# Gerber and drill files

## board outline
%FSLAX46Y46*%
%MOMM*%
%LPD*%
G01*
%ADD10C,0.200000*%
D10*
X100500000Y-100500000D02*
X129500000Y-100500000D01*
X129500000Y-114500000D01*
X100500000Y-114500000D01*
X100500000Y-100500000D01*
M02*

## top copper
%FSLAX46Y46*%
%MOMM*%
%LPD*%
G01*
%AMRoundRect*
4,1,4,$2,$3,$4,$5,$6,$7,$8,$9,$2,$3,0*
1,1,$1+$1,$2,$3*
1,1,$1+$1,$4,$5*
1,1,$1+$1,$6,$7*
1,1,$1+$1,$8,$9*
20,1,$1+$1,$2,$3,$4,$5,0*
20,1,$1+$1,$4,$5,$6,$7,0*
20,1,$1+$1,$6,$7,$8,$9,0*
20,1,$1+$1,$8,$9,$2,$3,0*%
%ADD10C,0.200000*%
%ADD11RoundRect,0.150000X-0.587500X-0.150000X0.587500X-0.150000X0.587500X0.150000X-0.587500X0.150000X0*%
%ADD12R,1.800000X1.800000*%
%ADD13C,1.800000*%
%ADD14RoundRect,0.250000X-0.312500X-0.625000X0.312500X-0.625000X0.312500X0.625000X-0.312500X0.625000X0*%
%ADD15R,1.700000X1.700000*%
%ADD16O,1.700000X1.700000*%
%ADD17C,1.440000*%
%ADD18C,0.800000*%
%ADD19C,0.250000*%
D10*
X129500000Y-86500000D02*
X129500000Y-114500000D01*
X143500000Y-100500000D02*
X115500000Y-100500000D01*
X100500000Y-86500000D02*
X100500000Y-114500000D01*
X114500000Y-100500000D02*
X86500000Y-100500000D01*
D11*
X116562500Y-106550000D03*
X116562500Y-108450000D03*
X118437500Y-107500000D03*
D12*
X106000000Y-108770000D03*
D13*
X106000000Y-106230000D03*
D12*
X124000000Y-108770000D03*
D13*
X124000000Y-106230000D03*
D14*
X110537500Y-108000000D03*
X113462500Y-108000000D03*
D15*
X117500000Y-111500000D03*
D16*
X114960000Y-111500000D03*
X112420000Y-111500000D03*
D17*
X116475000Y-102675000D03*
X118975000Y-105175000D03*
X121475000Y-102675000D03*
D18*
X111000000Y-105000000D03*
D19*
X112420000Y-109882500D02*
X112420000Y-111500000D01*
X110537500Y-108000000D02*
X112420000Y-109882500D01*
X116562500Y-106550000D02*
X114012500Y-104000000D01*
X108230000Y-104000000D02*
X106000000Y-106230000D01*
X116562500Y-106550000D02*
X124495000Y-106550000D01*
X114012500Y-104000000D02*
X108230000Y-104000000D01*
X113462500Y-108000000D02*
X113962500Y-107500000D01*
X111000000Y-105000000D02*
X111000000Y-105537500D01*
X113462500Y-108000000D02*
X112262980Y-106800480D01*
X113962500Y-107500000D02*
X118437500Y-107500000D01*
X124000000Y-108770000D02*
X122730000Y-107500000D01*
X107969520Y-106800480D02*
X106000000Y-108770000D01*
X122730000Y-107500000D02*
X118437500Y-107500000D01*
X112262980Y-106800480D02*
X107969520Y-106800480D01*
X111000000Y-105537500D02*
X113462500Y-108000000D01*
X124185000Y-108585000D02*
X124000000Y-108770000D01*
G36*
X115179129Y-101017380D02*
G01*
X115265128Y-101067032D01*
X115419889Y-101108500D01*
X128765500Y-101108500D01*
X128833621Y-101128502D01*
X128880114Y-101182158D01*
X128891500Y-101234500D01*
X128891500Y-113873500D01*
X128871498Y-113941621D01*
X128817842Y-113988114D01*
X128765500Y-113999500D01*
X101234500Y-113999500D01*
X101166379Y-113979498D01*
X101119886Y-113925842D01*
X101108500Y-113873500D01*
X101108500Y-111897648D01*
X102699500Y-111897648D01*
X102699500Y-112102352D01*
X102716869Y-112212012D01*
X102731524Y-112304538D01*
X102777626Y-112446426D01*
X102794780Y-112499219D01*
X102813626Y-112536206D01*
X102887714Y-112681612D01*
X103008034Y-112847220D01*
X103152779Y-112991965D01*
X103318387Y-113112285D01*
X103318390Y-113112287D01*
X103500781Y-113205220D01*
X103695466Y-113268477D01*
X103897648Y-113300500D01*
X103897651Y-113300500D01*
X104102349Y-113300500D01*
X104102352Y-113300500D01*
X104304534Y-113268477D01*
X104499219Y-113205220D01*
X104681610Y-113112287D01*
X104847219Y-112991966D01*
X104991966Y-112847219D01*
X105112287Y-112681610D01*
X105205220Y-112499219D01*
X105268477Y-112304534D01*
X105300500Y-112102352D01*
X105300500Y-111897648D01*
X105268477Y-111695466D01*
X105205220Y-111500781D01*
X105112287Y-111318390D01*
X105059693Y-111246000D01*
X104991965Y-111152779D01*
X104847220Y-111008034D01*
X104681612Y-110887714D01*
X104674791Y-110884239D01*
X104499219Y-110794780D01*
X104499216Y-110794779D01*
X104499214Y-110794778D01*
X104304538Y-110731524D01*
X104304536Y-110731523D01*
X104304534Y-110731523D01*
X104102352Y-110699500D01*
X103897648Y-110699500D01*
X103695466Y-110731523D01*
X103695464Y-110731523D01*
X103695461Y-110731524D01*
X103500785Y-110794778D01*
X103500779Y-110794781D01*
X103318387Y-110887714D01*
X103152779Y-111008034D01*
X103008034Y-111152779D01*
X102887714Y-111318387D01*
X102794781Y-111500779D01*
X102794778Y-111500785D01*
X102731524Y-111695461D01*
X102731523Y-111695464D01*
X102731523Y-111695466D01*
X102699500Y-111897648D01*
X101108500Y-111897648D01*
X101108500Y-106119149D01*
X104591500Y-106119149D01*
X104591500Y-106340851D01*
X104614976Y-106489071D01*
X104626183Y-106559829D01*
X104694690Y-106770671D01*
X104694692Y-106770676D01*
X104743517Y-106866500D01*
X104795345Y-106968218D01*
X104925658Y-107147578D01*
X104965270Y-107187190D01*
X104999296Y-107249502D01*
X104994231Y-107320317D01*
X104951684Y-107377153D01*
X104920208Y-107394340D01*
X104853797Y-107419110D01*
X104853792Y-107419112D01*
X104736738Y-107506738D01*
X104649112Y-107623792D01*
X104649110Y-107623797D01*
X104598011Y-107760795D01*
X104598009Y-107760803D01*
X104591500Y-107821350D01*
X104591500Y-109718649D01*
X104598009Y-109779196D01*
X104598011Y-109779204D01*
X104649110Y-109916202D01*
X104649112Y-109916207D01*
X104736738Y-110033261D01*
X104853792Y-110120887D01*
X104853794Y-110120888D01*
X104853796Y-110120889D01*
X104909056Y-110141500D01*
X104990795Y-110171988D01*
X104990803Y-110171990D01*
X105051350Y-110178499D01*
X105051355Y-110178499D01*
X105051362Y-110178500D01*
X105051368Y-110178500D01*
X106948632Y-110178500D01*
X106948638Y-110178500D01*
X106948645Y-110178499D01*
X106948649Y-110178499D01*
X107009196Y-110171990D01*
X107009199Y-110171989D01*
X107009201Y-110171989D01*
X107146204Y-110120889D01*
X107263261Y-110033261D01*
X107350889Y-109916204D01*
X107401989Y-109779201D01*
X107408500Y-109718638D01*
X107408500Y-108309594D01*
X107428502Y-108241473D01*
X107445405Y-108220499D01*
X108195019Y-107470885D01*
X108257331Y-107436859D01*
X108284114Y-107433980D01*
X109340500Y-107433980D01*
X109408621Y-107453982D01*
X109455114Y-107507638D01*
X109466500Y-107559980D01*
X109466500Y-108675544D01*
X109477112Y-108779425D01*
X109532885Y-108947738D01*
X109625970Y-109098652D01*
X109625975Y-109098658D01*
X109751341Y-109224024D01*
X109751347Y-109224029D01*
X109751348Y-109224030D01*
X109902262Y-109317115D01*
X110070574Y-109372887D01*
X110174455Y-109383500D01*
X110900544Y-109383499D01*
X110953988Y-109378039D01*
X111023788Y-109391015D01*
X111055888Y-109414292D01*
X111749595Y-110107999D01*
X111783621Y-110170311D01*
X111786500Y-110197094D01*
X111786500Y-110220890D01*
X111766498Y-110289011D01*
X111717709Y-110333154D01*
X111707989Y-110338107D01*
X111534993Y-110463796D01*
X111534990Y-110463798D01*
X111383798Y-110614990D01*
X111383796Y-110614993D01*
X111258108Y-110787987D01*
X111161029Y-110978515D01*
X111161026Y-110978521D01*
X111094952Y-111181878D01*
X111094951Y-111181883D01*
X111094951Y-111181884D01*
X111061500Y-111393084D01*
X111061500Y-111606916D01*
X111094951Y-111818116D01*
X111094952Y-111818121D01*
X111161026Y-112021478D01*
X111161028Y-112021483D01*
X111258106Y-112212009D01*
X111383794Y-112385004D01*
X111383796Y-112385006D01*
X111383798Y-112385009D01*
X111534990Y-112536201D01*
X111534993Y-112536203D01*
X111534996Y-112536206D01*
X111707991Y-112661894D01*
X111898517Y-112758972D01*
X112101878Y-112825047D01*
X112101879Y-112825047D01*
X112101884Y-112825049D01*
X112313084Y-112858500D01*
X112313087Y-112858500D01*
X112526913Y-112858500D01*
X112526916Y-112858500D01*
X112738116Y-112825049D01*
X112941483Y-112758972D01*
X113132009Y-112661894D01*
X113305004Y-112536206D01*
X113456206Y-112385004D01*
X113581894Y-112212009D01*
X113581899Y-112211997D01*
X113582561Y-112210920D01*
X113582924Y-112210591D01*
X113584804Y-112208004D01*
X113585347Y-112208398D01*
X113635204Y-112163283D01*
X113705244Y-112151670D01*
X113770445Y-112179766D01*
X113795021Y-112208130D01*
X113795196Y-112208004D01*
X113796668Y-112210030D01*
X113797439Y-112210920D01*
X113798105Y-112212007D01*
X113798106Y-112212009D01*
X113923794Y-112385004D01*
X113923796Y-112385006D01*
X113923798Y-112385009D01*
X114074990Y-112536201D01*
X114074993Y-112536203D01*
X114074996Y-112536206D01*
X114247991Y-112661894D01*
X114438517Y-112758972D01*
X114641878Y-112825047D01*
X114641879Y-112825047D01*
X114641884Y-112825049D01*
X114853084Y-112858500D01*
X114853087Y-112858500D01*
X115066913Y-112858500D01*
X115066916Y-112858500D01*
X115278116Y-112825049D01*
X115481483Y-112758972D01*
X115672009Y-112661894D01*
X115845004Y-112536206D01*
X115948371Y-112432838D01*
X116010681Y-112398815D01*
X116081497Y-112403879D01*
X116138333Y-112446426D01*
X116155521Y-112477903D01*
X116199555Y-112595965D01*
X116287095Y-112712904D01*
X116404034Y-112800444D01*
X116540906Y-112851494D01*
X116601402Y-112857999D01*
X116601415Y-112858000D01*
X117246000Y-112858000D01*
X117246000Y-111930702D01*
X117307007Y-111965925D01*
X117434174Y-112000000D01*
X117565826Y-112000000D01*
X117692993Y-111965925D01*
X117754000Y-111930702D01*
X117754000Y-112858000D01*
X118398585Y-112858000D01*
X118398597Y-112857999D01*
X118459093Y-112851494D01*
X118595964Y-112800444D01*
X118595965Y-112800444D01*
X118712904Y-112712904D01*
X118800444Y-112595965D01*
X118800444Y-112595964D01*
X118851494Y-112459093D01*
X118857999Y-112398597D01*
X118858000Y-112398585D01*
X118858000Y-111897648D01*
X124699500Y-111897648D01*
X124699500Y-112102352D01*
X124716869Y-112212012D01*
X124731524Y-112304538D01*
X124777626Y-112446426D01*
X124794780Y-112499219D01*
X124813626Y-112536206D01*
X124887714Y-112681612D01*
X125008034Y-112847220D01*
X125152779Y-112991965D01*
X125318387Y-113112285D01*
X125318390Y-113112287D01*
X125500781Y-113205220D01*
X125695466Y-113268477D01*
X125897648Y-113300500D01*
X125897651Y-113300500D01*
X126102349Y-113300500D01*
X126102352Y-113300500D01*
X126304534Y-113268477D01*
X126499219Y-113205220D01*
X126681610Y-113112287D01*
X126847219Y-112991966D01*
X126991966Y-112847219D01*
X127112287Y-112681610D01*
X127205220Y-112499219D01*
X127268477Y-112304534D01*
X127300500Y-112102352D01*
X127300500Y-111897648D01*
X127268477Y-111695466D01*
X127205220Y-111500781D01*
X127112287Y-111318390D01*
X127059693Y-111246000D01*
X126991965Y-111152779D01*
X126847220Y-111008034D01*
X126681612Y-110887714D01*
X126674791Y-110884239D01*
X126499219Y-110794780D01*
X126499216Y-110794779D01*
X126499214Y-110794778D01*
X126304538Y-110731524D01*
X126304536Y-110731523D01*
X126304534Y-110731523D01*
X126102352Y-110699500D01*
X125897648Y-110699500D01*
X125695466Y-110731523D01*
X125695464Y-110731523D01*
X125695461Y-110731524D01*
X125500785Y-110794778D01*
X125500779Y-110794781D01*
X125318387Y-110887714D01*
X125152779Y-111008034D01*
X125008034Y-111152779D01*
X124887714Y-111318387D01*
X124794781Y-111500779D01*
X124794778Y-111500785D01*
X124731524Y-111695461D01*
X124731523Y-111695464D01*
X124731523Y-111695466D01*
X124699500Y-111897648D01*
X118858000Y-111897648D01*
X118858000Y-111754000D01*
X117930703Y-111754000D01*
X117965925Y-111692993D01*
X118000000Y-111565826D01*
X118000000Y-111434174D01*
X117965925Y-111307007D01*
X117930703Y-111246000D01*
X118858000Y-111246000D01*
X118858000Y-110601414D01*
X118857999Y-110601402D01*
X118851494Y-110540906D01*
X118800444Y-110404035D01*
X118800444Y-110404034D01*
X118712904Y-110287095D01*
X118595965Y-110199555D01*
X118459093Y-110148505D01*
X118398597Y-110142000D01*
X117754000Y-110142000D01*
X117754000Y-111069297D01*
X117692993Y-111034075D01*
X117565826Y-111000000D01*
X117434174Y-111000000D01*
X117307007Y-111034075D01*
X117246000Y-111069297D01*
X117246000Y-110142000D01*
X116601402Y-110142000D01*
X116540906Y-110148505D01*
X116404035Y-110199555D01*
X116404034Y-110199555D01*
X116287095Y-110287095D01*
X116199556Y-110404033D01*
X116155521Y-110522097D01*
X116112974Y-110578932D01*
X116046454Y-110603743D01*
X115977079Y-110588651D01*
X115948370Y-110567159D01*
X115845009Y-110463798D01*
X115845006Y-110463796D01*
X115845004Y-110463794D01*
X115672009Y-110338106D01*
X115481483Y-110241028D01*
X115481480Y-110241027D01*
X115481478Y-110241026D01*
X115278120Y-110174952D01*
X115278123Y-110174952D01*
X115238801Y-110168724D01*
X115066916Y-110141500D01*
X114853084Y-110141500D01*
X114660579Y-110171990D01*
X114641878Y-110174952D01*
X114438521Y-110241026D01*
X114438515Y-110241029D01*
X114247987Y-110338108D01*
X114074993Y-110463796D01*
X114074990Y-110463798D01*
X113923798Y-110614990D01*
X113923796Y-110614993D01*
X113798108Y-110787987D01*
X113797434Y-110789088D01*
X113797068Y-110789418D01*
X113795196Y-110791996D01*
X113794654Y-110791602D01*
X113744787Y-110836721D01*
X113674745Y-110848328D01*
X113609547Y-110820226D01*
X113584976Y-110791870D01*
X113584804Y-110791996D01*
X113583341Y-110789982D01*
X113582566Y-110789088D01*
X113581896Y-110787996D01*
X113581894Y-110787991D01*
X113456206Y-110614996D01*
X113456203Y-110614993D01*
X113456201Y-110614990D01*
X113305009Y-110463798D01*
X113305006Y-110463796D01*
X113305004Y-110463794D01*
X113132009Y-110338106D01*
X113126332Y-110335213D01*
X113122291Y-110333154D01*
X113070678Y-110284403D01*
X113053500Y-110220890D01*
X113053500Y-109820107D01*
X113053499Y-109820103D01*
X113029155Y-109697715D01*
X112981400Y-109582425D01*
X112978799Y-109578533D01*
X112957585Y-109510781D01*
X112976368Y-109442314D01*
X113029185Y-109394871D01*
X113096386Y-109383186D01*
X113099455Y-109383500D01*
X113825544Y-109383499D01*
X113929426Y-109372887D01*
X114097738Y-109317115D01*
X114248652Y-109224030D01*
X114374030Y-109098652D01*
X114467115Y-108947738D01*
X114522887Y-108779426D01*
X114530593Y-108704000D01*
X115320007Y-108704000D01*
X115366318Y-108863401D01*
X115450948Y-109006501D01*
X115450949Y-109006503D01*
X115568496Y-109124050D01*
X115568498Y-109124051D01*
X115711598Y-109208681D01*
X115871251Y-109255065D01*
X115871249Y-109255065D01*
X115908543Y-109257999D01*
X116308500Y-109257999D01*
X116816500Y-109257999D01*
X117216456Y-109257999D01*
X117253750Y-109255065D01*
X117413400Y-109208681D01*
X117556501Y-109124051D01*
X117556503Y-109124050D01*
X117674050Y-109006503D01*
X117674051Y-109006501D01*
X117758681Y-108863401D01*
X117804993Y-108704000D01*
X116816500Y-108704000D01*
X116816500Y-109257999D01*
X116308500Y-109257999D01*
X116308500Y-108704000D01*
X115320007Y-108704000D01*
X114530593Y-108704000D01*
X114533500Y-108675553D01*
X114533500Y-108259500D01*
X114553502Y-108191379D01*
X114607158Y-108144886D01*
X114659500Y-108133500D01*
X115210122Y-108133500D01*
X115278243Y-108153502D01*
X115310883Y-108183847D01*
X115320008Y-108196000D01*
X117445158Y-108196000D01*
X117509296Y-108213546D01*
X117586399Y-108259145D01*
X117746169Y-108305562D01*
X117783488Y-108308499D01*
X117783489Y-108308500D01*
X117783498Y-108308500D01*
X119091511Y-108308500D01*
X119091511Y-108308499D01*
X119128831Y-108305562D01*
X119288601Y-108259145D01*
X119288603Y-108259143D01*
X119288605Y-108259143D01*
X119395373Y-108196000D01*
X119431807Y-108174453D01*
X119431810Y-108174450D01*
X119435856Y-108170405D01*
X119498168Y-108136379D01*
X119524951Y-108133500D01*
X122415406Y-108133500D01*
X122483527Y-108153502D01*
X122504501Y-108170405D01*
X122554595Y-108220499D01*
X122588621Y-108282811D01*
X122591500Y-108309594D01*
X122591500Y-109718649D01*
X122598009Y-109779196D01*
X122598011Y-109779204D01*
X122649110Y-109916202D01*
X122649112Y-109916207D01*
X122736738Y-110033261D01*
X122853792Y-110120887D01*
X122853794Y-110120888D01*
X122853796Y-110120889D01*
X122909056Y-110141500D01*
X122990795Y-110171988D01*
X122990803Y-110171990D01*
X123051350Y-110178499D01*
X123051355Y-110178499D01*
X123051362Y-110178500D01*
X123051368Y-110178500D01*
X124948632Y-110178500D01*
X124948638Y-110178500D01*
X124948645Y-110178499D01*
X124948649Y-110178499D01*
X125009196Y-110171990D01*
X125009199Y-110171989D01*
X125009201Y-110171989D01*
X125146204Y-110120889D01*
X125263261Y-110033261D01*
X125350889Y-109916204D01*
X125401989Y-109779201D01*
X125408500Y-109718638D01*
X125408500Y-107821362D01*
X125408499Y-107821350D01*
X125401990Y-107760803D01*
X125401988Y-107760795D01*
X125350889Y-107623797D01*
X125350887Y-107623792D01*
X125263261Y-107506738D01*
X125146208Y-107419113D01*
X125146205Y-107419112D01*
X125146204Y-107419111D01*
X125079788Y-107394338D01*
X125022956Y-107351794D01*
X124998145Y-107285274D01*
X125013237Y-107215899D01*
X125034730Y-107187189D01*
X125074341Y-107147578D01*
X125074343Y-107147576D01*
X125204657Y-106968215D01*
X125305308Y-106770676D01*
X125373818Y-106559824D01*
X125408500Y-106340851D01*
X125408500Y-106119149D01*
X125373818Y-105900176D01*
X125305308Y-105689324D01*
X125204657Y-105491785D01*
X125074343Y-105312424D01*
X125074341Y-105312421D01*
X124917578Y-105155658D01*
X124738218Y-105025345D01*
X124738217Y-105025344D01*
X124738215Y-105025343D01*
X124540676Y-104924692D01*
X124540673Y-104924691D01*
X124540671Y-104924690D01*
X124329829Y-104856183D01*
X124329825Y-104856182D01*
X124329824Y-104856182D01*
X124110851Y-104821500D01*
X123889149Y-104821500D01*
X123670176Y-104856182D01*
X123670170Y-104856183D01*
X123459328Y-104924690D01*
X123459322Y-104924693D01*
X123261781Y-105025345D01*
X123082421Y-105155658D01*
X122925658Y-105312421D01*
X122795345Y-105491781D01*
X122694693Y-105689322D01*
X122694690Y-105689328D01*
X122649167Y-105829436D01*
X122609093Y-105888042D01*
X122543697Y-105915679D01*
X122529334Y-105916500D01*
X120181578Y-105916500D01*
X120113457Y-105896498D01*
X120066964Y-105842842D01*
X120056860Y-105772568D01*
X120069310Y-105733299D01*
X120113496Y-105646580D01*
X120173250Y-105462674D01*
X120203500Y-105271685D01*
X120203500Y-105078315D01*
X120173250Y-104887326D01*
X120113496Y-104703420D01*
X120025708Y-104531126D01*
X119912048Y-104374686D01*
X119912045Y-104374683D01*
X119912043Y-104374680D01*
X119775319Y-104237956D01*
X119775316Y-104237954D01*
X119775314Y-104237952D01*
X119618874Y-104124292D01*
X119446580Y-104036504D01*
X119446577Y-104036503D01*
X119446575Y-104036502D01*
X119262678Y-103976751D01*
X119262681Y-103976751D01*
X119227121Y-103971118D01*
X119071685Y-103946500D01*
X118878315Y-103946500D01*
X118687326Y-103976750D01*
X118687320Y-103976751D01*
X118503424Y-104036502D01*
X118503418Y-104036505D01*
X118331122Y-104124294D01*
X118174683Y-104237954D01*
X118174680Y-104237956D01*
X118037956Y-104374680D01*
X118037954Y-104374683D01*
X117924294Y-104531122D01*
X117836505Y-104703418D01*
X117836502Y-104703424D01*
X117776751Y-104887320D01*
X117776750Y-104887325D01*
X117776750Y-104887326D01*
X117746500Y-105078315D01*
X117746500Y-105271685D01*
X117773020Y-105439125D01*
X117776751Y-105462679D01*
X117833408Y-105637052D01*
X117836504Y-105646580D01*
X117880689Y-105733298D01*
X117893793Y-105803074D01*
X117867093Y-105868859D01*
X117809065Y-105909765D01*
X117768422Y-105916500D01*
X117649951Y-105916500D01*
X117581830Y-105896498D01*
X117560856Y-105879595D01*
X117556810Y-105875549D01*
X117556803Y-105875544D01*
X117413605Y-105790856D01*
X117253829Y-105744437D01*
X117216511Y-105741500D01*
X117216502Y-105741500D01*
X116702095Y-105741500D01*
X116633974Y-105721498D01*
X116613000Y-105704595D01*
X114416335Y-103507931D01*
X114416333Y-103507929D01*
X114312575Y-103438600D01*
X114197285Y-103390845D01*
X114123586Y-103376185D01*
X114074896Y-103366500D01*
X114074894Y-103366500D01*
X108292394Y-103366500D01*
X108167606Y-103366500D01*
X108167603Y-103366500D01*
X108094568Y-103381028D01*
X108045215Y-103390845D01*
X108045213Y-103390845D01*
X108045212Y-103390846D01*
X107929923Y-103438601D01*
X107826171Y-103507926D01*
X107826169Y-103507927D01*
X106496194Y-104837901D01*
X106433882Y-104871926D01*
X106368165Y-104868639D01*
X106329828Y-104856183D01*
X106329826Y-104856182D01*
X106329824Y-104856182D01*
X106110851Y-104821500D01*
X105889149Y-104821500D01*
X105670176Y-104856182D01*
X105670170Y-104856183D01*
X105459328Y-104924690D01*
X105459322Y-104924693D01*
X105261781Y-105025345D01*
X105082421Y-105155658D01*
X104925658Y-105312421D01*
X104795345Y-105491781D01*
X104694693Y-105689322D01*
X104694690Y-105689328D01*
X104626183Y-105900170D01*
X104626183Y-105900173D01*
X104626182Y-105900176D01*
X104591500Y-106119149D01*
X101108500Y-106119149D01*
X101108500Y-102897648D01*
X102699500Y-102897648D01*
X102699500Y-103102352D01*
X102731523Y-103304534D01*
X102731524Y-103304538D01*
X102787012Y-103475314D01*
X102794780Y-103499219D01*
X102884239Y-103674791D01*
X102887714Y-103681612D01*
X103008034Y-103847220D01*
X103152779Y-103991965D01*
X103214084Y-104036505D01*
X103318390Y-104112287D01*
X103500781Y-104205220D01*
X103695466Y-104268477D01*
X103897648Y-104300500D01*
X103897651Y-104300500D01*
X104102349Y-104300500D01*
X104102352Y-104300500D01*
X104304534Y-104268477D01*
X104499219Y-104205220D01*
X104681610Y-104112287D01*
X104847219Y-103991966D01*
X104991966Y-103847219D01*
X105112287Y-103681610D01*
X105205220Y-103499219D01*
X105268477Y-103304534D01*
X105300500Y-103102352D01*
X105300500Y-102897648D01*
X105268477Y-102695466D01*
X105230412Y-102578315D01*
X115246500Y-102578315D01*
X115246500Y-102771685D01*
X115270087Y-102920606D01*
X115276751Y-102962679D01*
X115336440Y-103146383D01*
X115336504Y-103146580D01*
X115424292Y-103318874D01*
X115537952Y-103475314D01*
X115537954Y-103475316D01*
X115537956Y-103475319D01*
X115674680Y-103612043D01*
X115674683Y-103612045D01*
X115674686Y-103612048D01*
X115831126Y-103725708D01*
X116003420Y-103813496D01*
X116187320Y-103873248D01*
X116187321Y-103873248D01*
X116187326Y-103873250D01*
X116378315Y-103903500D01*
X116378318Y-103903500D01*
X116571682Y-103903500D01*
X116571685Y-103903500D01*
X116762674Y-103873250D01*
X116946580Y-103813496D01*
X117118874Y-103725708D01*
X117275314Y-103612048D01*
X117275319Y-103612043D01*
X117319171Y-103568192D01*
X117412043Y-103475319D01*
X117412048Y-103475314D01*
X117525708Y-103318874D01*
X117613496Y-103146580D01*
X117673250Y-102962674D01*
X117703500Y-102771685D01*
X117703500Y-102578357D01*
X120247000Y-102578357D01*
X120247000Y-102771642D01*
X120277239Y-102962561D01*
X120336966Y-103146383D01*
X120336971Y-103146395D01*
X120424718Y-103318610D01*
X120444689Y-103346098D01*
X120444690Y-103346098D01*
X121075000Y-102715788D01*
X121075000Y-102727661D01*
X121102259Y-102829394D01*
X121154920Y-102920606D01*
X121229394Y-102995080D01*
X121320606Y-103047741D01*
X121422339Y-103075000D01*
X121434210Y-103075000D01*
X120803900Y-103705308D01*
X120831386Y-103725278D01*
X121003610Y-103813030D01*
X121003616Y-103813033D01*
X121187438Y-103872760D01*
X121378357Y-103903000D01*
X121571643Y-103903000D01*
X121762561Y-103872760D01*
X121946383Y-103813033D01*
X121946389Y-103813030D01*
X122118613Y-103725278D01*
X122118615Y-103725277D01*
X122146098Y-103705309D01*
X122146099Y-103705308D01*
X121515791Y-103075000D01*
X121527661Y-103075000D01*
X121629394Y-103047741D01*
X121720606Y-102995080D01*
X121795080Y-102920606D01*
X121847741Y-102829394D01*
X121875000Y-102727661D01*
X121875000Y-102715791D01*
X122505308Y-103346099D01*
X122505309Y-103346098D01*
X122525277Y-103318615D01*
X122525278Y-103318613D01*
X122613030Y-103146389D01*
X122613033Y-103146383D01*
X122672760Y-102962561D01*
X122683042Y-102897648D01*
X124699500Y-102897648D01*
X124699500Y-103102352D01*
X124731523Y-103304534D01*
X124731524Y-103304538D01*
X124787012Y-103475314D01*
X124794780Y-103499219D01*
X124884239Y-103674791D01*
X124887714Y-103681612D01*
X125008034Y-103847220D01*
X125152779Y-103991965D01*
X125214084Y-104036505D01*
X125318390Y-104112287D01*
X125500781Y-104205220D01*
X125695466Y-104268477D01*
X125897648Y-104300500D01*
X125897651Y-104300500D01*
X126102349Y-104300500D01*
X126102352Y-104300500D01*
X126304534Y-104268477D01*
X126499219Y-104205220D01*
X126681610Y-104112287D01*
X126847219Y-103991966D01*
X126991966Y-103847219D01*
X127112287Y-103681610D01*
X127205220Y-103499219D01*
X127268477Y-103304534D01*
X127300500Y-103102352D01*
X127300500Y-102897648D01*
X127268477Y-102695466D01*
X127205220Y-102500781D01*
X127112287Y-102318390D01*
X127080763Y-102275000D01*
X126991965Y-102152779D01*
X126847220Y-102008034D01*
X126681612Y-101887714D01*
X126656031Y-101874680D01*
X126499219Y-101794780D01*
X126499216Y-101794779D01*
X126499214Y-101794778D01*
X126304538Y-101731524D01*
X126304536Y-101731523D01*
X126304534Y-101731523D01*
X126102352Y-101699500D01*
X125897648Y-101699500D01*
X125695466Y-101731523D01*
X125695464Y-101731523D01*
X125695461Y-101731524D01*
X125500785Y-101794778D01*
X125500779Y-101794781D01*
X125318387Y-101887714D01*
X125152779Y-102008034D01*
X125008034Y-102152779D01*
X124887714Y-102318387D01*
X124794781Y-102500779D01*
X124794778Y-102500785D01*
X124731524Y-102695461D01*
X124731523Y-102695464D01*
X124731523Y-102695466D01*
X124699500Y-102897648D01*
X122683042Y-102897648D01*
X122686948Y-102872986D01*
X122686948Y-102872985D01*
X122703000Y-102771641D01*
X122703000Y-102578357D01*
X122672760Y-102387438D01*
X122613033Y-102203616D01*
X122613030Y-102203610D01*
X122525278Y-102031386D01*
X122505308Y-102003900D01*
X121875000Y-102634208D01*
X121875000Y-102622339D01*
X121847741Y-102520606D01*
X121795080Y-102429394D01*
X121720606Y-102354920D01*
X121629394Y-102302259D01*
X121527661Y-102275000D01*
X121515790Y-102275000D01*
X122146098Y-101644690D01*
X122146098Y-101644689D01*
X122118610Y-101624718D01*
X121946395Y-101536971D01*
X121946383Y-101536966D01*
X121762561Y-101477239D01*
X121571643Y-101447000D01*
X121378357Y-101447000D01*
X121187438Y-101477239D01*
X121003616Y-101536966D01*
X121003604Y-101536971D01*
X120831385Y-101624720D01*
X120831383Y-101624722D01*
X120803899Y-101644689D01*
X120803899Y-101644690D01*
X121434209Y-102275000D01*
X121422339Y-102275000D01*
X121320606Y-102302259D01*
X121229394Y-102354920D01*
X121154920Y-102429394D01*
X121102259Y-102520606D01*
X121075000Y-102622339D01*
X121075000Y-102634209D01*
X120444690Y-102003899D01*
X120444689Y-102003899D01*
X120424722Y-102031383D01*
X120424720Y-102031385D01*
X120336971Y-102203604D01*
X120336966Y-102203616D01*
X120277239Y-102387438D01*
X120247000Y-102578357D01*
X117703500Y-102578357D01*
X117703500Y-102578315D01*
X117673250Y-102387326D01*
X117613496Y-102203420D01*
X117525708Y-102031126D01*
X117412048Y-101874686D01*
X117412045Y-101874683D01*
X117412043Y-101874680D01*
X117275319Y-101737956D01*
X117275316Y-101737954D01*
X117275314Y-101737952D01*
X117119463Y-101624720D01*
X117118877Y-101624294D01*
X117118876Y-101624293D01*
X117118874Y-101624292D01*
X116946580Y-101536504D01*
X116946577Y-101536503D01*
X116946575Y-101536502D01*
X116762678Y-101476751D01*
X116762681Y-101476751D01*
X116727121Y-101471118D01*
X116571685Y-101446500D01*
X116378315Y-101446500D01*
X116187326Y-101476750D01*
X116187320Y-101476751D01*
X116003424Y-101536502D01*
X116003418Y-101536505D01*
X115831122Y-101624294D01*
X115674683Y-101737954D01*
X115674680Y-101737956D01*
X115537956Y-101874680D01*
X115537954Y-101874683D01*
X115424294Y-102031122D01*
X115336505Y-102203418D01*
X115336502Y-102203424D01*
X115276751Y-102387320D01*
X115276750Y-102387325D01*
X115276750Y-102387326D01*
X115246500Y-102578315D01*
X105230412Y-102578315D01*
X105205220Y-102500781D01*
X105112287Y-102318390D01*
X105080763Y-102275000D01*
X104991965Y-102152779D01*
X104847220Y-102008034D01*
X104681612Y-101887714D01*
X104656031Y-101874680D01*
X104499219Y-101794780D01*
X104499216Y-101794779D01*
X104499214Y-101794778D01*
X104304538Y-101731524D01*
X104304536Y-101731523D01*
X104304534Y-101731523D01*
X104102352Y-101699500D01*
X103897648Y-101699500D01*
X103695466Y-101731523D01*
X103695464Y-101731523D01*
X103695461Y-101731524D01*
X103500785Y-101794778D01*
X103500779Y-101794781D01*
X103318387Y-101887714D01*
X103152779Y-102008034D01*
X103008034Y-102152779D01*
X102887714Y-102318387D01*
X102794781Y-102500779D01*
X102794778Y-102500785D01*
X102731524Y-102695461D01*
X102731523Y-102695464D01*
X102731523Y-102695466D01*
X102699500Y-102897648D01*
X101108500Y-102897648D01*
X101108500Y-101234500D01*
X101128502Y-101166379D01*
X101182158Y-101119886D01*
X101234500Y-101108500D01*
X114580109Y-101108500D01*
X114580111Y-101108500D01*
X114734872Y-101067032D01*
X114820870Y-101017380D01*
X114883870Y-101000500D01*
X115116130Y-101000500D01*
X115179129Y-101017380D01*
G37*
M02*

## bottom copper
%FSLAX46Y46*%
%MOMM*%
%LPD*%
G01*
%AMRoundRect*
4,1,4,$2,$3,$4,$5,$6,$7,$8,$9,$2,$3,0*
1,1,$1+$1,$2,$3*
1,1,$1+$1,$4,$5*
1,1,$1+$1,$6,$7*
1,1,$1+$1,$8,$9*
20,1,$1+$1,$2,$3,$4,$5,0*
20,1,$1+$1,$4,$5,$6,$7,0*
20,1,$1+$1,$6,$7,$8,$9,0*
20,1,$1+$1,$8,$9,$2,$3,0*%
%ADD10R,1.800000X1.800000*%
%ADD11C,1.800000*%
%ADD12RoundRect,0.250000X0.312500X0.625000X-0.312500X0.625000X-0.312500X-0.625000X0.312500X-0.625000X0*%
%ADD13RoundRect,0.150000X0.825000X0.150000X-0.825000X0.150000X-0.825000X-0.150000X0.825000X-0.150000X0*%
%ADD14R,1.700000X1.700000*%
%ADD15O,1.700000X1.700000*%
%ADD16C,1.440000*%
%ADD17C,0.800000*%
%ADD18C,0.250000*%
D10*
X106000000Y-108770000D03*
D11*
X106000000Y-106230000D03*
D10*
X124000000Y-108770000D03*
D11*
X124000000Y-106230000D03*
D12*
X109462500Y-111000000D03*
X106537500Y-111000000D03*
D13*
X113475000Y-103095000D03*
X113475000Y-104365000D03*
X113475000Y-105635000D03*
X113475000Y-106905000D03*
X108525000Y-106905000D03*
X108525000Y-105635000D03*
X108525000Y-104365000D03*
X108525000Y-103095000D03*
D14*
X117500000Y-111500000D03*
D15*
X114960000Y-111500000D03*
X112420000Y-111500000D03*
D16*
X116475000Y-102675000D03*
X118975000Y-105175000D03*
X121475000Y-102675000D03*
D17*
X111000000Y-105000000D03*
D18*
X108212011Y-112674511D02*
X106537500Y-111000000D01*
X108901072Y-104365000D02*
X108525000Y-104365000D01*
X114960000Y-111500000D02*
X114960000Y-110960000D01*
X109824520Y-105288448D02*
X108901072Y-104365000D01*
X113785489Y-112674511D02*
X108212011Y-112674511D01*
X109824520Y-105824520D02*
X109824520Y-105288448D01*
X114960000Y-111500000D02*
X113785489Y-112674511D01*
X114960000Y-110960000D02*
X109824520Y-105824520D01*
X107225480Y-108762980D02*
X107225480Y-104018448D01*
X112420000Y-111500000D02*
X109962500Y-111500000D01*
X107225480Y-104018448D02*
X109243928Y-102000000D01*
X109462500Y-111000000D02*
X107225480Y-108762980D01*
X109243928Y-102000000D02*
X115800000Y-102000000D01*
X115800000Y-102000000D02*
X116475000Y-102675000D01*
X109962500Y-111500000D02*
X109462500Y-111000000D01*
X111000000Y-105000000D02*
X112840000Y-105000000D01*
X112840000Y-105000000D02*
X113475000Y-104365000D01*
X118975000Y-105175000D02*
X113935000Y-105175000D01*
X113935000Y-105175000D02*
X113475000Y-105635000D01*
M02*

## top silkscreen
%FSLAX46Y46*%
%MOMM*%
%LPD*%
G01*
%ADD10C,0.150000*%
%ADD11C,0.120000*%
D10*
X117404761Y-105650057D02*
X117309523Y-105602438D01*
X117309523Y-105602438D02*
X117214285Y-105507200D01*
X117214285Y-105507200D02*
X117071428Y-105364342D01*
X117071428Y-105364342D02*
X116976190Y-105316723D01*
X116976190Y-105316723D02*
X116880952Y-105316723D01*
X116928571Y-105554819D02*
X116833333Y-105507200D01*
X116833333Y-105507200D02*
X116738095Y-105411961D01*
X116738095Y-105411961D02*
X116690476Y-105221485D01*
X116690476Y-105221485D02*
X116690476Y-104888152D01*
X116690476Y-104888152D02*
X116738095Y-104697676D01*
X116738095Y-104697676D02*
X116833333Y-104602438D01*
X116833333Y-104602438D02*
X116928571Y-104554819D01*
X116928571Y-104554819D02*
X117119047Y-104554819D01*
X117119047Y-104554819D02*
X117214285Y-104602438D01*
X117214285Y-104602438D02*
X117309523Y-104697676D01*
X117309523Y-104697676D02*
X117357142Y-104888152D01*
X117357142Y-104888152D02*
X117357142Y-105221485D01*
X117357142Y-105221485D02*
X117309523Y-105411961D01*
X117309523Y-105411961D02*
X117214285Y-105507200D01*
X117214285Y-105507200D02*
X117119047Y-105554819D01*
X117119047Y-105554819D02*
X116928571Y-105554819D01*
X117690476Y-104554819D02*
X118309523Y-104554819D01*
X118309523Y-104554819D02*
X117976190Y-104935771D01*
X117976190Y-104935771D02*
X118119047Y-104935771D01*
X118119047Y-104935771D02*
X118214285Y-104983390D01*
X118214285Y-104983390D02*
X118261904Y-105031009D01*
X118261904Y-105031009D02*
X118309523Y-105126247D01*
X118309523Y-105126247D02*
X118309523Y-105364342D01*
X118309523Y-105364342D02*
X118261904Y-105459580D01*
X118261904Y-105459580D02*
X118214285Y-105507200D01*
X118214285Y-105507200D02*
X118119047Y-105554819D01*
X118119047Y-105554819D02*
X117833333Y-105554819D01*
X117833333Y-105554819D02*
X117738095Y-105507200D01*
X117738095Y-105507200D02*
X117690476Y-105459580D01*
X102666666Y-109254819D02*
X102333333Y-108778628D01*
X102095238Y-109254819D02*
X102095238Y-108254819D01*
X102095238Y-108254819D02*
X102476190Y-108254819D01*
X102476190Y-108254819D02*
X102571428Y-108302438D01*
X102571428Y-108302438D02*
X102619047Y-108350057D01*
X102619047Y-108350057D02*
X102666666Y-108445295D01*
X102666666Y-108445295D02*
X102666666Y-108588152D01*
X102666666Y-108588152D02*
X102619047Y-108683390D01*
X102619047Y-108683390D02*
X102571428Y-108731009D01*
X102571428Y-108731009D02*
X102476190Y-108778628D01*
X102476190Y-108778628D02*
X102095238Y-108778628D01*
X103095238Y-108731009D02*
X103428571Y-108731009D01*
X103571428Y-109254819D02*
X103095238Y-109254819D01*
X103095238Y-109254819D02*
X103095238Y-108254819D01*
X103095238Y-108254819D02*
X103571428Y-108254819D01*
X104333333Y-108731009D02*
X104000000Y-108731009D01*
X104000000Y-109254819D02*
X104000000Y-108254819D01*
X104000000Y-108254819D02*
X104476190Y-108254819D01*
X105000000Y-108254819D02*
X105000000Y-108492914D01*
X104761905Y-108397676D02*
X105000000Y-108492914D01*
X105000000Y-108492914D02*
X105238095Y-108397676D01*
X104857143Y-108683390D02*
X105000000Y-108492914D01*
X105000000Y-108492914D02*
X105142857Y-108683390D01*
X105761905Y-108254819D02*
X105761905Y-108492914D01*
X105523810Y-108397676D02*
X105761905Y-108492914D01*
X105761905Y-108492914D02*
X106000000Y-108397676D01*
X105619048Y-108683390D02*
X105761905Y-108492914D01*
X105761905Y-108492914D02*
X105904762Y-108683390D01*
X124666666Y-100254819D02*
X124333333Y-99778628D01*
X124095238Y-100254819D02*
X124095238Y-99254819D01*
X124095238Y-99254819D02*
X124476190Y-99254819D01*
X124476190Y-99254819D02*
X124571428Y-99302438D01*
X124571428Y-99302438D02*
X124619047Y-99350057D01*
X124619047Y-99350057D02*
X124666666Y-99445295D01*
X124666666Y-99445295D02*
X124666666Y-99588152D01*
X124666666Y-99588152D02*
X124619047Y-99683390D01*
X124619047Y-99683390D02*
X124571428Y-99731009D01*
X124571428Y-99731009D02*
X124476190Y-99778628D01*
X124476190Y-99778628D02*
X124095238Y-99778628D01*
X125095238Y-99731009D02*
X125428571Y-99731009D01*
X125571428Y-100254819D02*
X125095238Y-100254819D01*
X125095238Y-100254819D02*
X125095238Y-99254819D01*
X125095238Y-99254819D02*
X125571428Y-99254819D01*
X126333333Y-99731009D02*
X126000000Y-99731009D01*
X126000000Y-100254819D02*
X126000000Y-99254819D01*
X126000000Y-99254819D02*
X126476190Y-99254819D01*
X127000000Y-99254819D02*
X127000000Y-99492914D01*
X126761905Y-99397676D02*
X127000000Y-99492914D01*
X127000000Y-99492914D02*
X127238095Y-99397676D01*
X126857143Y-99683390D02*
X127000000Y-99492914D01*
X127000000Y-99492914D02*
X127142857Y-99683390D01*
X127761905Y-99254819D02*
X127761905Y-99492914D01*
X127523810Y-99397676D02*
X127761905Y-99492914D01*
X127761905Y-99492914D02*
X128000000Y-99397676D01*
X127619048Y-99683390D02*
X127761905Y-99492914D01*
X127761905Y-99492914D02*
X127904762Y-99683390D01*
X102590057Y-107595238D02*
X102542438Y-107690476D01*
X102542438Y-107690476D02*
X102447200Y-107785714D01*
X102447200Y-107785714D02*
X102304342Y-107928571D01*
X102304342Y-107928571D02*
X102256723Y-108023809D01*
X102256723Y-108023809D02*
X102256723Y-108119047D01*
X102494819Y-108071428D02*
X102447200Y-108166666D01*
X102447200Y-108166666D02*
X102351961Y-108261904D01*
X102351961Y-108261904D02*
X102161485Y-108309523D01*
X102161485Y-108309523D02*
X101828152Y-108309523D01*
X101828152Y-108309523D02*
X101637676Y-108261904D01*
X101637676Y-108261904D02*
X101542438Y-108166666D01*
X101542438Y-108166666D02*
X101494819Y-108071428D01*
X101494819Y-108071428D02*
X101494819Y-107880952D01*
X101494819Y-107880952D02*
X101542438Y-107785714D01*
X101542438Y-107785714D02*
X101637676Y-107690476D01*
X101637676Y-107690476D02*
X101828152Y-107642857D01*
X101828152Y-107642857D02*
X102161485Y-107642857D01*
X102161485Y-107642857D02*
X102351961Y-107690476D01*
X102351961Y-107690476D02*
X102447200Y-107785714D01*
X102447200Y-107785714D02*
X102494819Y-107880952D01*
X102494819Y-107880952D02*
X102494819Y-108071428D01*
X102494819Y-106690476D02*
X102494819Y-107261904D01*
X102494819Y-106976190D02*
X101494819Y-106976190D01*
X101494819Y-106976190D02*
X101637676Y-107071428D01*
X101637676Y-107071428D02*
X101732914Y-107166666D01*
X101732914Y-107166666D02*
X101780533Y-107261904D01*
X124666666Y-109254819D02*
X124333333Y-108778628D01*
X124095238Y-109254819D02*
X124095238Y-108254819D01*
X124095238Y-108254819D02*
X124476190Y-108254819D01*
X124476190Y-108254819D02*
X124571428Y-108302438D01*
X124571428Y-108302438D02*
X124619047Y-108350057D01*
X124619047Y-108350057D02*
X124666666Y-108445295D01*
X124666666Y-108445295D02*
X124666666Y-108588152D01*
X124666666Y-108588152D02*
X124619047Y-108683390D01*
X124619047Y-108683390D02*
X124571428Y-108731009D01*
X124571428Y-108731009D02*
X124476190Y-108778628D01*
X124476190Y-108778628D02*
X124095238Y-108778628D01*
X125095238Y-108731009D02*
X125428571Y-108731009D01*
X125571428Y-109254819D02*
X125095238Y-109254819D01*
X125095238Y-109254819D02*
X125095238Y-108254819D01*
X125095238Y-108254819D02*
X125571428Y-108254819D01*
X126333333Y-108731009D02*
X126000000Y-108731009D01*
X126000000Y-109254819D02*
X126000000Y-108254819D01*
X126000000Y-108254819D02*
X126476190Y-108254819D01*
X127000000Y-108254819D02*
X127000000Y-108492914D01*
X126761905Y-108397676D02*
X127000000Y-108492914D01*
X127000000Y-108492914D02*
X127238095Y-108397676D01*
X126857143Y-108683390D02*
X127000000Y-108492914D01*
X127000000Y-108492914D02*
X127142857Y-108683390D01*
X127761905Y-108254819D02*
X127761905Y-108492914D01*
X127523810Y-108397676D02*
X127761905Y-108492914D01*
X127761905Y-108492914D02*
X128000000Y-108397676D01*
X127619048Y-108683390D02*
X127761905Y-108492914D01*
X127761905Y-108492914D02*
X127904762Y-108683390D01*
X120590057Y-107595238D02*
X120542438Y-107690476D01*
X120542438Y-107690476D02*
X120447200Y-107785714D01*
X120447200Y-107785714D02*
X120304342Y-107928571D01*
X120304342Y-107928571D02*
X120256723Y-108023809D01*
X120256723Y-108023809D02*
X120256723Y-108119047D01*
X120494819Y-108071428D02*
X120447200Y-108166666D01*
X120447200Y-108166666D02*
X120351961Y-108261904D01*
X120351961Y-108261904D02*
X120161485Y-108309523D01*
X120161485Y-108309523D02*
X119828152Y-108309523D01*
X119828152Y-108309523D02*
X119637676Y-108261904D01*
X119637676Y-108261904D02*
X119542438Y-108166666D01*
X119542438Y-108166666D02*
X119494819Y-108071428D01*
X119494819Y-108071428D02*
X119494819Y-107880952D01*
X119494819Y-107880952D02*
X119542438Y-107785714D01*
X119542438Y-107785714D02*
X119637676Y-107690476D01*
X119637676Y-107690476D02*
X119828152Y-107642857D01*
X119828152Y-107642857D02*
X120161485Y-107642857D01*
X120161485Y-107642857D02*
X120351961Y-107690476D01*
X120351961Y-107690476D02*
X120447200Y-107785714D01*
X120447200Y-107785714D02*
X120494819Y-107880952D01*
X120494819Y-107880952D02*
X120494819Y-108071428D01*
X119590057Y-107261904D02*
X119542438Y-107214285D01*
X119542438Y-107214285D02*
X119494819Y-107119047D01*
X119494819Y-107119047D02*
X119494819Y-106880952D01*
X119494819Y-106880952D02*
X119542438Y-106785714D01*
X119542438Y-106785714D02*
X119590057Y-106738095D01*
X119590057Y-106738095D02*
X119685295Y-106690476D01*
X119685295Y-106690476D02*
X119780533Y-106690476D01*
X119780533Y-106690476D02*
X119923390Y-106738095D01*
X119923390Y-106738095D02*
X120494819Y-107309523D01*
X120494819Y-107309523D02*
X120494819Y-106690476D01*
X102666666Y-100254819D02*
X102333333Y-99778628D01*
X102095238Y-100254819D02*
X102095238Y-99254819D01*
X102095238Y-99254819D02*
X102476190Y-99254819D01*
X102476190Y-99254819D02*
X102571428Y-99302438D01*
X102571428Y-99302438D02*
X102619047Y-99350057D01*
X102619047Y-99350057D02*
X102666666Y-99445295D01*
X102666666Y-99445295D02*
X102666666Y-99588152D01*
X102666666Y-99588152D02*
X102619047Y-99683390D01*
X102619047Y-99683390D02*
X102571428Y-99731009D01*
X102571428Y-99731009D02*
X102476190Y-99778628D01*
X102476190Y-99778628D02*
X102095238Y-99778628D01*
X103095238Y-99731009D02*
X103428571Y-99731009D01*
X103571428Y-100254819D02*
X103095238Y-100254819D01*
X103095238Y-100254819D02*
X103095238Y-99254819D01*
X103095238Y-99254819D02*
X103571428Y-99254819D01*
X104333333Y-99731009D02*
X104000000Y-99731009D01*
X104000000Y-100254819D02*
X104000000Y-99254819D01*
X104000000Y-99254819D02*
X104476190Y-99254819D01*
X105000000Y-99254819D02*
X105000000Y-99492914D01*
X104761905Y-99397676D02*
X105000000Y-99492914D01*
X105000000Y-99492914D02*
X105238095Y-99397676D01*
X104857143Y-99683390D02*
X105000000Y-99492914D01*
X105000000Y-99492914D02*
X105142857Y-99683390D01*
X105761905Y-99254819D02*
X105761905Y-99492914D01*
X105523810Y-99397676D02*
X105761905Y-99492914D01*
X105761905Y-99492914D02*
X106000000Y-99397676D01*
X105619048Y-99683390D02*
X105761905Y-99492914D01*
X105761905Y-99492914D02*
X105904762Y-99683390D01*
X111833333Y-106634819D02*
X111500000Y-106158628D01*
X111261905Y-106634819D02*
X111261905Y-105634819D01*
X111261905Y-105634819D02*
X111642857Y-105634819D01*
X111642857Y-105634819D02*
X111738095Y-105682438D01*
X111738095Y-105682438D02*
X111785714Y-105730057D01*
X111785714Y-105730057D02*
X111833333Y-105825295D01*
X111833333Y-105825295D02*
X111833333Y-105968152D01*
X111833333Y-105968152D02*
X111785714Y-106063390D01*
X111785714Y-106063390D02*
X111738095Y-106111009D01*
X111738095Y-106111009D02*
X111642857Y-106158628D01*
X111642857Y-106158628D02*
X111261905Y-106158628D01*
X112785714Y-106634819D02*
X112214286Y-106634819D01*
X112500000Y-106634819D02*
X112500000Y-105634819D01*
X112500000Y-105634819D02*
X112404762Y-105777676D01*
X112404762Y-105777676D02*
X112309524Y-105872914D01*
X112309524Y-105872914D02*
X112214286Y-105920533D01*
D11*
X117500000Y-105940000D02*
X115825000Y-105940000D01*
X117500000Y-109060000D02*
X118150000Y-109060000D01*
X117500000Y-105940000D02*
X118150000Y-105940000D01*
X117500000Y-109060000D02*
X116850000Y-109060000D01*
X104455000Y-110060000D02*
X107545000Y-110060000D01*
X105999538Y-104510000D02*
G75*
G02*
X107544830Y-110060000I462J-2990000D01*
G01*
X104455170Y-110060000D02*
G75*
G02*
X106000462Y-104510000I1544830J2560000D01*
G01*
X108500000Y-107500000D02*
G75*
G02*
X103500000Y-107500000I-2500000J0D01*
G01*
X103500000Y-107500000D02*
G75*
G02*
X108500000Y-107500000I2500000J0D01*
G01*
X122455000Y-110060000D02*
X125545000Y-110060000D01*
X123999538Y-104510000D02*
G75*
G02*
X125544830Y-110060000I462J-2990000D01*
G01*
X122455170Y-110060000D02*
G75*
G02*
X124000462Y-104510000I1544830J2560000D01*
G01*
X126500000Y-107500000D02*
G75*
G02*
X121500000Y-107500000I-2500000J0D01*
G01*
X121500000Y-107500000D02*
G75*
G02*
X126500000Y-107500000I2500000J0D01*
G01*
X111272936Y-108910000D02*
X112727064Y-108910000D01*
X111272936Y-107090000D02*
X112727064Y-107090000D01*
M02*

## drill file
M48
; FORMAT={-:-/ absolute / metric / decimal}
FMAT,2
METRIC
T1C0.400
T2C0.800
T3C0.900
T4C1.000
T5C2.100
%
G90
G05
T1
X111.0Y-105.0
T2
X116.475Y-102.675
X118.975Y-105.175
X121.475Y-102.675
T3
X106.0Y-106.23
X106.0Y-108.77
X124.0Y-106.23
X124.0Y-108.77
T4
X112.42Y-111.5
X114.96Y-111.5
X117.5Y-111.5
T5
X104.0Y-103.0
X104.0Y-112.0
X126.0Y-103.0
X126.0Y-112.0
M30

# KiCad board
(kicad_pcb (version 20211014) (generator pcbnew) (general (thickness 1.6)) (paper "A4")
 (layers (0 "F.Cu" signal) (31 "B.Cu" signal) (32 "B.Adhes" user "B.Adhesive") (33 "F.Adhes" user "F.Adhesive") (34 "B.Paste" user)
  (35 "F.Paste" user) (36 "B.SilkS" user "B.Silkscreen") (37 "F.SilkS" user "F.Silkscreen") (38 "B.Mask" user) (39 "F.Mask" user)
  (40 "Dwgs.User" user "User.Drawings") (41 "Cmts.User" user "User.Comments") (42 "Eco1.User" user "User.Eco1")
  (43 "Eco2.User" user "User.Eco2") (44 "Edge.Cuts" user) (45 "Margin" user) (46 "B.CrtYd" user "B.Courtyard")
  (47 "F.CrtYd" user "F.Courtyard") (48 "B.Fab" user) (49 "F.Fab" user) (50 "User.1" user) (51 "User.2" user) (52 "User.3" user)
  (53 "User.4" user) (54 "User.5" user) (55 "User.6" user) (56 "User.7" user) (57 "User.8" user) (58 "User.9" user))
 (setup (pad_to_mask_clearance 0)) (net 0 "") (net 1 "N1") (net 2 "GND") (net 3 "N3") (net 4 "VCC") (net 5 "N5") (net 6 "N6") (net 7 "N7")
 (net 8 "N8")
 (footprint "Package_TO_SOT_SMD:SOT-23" (layer "F.Cu") (at 117.5 107.5)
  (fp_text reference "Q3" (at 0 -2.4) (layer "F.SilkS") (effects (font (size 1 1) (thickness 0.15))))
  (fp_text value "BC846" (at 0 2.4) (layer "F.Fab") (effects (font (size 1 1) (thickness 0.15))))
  (fp_line (start 0 -1.56) (end -1.675 -1.56) (layer "F.SilkS") (width 0.12))
  (fp_line (start 0 1.56) (end 0.65 1.56) (layer "F.SilkS") (width 0.12))
  (fp_line (start 0 -1.56) (end 0.65 -1.56) (layer "F.SilkS") (width 0.12))
  (fp_line (start 0 1.56) (end -0.65 1.56) (layer "F.SilkS") (width 0.12))
  (pad "1" smd roundrect (at -0.9375 -0.95) (size 1.475 0.6) (layers "F.Cu" "F.Paste" "F.Mask") (roundrect_rratio 0.25) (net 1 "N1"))
  (pad "2" smd roundrect (at -0.9375 0.95) (size 1.475 0.6) (layers "F.Cu" "F.Paste" "F.Mask") (roundrect_rratio 0.25) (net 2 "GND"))
  (pad "3" smd roundrect (at 0.9375 0) (size 1.475 0.6) (layers "F.Cu" "F.Paste" "F.Mask") (roundrect_rratio 0.25) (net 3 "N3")))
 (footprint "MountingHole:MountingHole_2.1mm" (layer "F.Cu") (at 104 112)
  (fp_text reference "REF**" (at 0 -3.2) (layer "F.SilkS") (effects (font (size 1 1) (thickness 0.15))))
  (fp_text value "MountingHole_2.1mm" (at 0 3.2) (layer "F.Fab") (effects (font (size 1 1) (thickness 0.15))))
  (pad "" np_thru_hole circle (at 0 0) (size 2.1 2.1) (drill 2.1) (layers *.Cu *.Mask)))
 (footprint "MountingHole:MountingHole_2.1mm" (layer "F.Cu") (at 126 103)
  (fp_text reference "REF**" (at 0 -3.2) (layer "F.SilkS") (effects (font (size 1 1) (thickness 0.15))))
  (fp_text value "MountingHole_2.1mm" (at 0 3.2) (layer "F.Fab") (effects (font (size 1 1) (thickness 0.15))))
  (pad "" np_thru_hole circle (at 0 0) (size 2.1 2.1) (drill 2.1) (layers *.Cu *.Mask)))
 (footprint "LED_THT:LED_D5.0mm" (layer "F.Cu") (at 106 108.77 90)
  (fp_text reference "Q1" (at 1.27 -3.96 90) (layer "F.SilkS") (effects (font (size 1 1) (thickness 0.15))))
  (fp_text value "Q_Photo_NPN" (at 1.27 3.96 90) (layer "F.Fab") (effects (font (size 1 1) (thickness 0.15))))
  (fp_line (start -1.29 -1.545) (end -1.29 1.545) (layer "F.SilkS") (width 0.12))
  (fp_arc (start 4.26 -0.000462) (mid 2.072002 2.880433) (end -1.29 1.54483) (layer "F.SilkS") (width 0.12))
  (fp_arc (start -1.29 -1.54483) (mid 2.072002 -2.880433) (end 4.26 0.000462) (layer "F.SilkS") (width 0.12))
  (fp_circle (center 1.27 0) (end 3.77 0) (layer "F.SilkS") (width 0.12) (fill none))
  (pad "1" thru_hole rect (at 0 0 90) (size 1.8 1.8) (drill 0.9) (layers *.Cu *.Mask) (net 3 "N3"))
  (pad "2" thru_hole circle (at 2.54 0 90) (size 1.8 1.8) (drill 0.9) (layers *.Cu *.Mask) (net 1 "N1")))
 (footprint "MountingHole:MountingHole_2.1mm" (layer "F.Cu") (at 126 112)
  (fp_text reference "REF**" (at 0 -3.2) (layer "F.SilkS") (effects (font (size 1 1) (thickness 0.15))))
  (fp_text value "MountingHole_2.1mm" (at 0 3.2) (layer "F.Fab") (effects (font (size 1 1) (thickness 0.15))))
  (pad "" np_thru_hole circle (at 0 0) (size 2.1 2.1) (drill 2.1) (layers *.Cu *.Mask)))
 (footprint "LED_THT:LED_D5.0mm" (layer "F.Cu") (at 124 108.77 90)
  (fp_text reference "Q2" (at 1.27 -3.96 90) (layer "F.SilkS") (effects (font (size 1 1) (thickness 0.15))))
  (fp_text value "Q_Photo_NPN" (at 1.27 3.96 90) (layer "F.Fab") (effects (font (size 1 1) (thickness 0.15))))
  (fp_line (start -1.29 -1.545) (end -1.29 1.545) (layer "F.SilkS") (width 0.12))
  (fp_arc (start 4.26 -0.000462) (mid 2.072002 2.880433) (end -1.29 1.54483) (layer "F.SilkS") (width 0.12))
  (fp_arc (start -1.29 -1.54483) (mid 2.072002 -2.880433) (end 4.26 0.000462) (layer "F.SilkS") (width 0.12))
  (fp_circle (center 1.27 0) (end 3.77 0) (layer "F.SilkS") (width 0.12) (fill none))
  (pad "1" thru_hole rect (at 0 0 90) (size 1.8 1.8) (drill 0.9) (layers *.Cu *.Mask) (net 3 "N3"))
  (pad "2" thru_hole circle (at 2.54 0 90) (size 1.8 1.8) (drill 0.9) (layers *.Cu *.Mask) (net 1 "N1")))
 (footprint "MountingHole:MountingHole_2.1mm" (layer "F.Cu") (at 104 103)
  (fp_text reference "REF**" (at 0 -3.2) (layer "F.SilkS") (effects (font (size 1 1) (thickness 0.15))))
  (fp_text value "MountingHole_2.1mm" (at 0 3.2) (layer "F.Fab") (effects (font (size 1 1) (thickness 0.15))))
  (pad "" np_thru_hole circle (at 0 0) (size 2.1 2.1) (drill 2.1) (layers *.Cu *.Mask)))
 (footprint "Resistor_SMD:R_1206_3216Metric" (layer "F.Cu") (at 112 108)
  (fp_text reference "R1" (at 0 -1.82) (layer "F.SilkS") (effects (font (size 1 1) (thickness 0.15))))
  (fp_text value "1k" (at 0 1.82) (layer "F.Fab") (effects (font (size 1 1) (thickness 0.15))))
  (fp_line (start -0.727064 0.91) (end 0.727064 0.91) (layer "F.SilkS") (width 0.12))
  (fp_line (start -0.727064 -0.91) (end 0.727064 -0.91) (layer "F.SilkS") (width 0.12))
  (pad "1" smd roundrect (at -1.4625 0) (size 1.125 1.75) (layers "F.Cu" "F.Paste" "F.Mask") (roundrect_rratio 0.2222222222) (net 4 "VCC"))
  (pad "2" smd roundrect (at 1.4625 0) (size 1.125 1.75) (layers "F.Cu" "F.Paste" "F.Mask") (roundrect_rratio 0.2222222222) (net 3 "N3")))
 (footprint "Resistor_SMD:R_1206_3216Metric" (layer "B.Cu") (at 108 111 180)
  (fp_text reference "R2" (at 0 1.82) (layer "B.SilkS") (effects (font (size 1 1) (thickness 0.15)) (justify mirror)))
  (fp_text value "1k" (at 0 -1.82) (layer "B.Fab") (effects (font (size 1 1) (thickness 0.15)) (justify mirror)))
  (pad "1" smd roundrect (at -1.4625 0 180) (size 1.125 1.75) (layers "B.Cu" "B.Paste" "B.Mask") (roundrect_rratio 0.2222222222)
   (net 4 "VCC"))
  (pad "2" smd roundrect (at 1.4625 0 180) (size 1.125 1.75) (layers "B.Cu" "B.Paste" "B.Mask") (roundrect_rratio 0.2222222222) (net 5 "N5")))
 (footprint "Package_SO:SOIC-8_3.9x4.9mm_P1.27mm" (layer "B.Cu") (at 111 105 180)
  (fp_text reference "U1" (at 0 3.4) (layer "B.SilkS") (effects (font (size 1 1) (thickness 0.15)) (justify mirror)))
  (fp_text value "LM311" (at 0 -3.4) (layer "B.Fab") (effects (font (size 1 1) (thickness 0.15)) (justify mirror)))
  (pad "1" smd roundrect (at -2.475 1.905 180) (size 1.95 0.6) (layers "B.Cu" "B.Paste" "B.Mask") (roundrect_rratio 0.25) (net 2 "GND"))
  (pad "2" smd roundrect (at -2.475 0.635 180) (size 1.95 0.6) (layers "B.Cu" "B.Paste" "B.Mask") (roundrect_rratio 0.25) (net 3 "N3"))
  (pad "3" smd roundrect (at -2.475 -0.635 180) (size 1.95 0.6) (layers "B.Cu" "B.Paste" "B.Mask") (roundrect_rratio 0.25) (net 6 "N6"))
  (pad "4" smd roundrect (at -2.475 -1.905 180) (size 1.95 0.6) (layers "B.Cu" "B.Paste" "B.Mask") (roundrect_rratio 0.25) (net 2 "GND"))
  (pad "5" smd roundrect (at 2.475 -1.905 180) (size 1.95 0.6) (layers "B.Cu" "B.Paste" "B.Mask") (roundrect_rratio 0.25) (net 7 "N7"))
  (pad "6" smd roundrect (at 2.475 -0.635 180) (size 1.95 0.6) (layers "B.Cu" "B.Paste" "B.Mask") (roundrect_rratio 0.25) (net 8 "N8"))
  (pad "7" smd roundrect (at 2.475 0.635 180) (size 1.95 0.6) (layers "B.Cu" "B.Paste" "B.Mask") (roundrect_rratio 0.25) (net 5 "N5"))
  (pad "8" smd roundrect (at 2.475 1.905 180) (size 1.95 0.6) (layers "B.Cu" "B.Paste" "B.Mask") (roundrect_rratio 0.25) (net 4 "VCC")))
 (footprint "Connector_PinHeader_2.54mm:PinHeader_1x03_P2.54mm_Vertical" (layer "B.Cu") (at 117.5 111.5 90)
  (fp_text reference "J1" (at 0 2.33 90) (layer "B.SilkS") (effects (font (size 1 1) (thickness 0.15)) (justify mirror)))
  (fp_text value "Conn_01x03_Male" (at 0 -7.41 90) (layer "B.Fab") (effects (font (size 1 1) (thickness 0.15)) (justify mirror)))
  (pad "1" thru_hole rect (at 0 0 90) (size 1.7 1.7) (drill 1) (layers *.Cu *.Mask) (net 2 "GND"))
  (pad "2" thru_hole oval (at 0 -2.54 90) (size 1.7 1.7) (drill 1) (layers *.Cu *.Mask) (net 5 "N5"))
  (pad "3" thru_hole oval (at 0 -5.08 90) (size 1.7 1.7) (drill 1) (layers *.Cu *.Mask) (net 4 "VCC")))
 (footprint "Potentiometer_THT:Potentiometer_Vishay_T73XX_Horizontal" (layer "B.Cu") (at 116.475 102.675 -90)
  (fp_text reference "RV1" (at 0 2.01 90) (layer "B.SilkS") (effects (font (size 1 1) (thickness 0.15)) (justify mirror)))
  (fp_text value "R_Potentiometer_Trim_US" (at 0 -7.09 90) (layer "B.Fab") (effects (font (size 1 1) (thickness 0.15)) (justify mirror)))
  (pad "1" thru_hole circle (at 0 0 270) (size 1.44 1.44) (drill 0.8) (layers *.Cu *.Mask) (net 4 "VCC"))
  (pad "2" thru_hole circle (at 2.5 -2.5 270) (size 1.44 1.44) (drill 0.8) (layers *.Cu *.Mask) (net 6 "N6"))
  (pad "3" thru_hole circle (at 0 -5 270) (size 1.44 1.44) (drill 0.8) (layers *.Cu *.Mask) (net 2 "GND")))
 (gr_rect (start 100.5 100.5) (end 129.5 114.5) (layer "Edge.Cuts") (width 0.2) (fill none))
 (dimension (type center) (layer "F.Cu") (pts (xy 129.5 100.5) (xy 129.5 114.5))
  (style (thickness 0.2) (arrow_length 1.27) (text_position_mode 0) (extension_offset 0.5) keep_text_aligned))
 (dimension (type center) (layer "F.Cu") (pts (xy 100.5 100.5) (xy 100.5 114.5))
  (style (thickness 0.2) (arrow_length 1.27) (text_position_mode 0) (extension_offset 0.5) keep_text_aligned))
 (segment (start 108.212011 112.674511) (end 106.5375 111) (width 0.25) (layer "B.Cu") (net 5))
 (segment (start 108.901072 104.365) (end 108.525 104.365) (width 0.25) (layer "B.Cu") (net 5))
 (segment (start 114.96 111.5) (end 114.96 110.96) (width 0.25) (layer "B.Cu") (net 5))
 (segment (start 109.82452 105.288448) (end 108.901072 104.365) (width 0.25) (layer "B.Cu") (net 5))
 (segment (start 113.785489 112.674511) (end 108.212011 112.674511) (width 0.25) (layer "B.Cu") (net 5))
 (segment (start 109.82452 105.82452) (end 109.82452 105.288448) (width 0.25) (layer "B.Cu") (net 5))
 (segment (start 114.96 111.5) (end 113.785489 112.674511) (width 0.25) (layer "B.Cu") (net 5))
 (segment (start 114.96 110.96) (end 109.82452 105.82452) (width 0.25) (layer "B.Cu") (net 5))
 (segment (start 112.42 109.8825) (end 112.42 111.5) (width 0.25) (layer "F.Cu") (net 4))
 (segment (start 110.5375 108) (end 112.42 109.8825) (width 0.25) (layer "F.Cu") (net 4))
 (segment (start 107.22548 108.76298) (end 107.22548 104.018448) (width 0.25) (layer "B.Cu") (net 4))
 (segment (start 112.42 111.5) (end 109.9625 111.5) (width 0.25) (layer "B.Cu") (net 4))
 (segment (start 107.22548 104.018448) (end 109.243928 102) (width 0.25) (layer "B.Cu") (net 4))
 (segment (start 109.4625 111) (end 107.22548 108.76298) (width 0.25) (layer "B.Cu") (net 4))
 (segment (start 109.243928 102) (end 115.8 102) (width 0.25) (layer "B.Cu") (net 4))
 (segment (start 115.8 102) (end 116.475 102.675) (width 0.25) (layer "B.Cu") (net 4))
 (segment (start 109.9625 111.5) (end 109.4625 111) (width 0.25) (layer "B.Cu") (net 4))
 (segment (start 116.5625 106.55) (end 114.0125 104) (width 0.25) (layer "F.Cu") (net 1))
 (segment (start 108.23 104) (end 106 106.23) (width 0.25) (layer "F.Cu") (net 1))
 (segment (start 116.5625 106.55) (end 124.495 106.55) (width 0.25) (layer "F.Cu") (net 1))
 (segment (start 114.0125 104) (end 108.23 104) (width 0.25) (layer "F.Cu") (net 1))
 (segment (start 113.4625 108) (end 113.9625 107.5) (width 0.25) (layer "F.Cu") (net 3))
 (segment (start 111 105) (end 111 105.5375) (width 0.25) (layer "F.Cu") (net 3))
 (segment (start 113.4625 108) (end 112.26298 106.80048) (width 0.25) (layer "F.Cu") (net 3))
 (segment (start 113.9625 107.5) (end 118.4375 107.5) (width 0.25) (layer "F.Cu") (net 3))
 (segment (start 124 108.77) (end 122.73 107.5) (width 0.25) (layer "F.Cu") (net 3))
 (segment (start 107.96952 106.80048) (end 106 108.77) (width 0.25) (layer "F.Cu") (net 3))
 (segment (start 122.73 107.5) (end 118.4375 107.5) (width 0.25) (layer "F.Cu") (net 3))
 (segment (start 112.26298 106.80048) (end 107.96952 106.80048) (width 0.25) (layer "F.Cu") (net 3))
 (segment (start 111 105.5375) (end 113.4625 108) (width 0.25) (layer "F.Cu") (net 3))
 (segment (start 124.185 108.585) (end 124 108.77) (width 0.25) (layer "F.Cu") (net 3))
 (via (at 111 105) (size 0.8) (drill 0.4) (layers "F.Cu" "B.Cu") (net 3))
 (segment (start 111 105) (end 112.84 105) (width 0.25) (layer "B.Cu") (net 3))
 (segment (start 112.84 105) (end 113.475 104.365) (width 0.25) (layer "B.Cu") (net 3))
 (segment (start 118.975 105.175) (end 113.935 105.175) (width 0.25) (layer "B.Cu") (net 6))
 (segment (start 113.935 105.175) (end 113.475 105.635) (width 0.25) (layer "B.Cu") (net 6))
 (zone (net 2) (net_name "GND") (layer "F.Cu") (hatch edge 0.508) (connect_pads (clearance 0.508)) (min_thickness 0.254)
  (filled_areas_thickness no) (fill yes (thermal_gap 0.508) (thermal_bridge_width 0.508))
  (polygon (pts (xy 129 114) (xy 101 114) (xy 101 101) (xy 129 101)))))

